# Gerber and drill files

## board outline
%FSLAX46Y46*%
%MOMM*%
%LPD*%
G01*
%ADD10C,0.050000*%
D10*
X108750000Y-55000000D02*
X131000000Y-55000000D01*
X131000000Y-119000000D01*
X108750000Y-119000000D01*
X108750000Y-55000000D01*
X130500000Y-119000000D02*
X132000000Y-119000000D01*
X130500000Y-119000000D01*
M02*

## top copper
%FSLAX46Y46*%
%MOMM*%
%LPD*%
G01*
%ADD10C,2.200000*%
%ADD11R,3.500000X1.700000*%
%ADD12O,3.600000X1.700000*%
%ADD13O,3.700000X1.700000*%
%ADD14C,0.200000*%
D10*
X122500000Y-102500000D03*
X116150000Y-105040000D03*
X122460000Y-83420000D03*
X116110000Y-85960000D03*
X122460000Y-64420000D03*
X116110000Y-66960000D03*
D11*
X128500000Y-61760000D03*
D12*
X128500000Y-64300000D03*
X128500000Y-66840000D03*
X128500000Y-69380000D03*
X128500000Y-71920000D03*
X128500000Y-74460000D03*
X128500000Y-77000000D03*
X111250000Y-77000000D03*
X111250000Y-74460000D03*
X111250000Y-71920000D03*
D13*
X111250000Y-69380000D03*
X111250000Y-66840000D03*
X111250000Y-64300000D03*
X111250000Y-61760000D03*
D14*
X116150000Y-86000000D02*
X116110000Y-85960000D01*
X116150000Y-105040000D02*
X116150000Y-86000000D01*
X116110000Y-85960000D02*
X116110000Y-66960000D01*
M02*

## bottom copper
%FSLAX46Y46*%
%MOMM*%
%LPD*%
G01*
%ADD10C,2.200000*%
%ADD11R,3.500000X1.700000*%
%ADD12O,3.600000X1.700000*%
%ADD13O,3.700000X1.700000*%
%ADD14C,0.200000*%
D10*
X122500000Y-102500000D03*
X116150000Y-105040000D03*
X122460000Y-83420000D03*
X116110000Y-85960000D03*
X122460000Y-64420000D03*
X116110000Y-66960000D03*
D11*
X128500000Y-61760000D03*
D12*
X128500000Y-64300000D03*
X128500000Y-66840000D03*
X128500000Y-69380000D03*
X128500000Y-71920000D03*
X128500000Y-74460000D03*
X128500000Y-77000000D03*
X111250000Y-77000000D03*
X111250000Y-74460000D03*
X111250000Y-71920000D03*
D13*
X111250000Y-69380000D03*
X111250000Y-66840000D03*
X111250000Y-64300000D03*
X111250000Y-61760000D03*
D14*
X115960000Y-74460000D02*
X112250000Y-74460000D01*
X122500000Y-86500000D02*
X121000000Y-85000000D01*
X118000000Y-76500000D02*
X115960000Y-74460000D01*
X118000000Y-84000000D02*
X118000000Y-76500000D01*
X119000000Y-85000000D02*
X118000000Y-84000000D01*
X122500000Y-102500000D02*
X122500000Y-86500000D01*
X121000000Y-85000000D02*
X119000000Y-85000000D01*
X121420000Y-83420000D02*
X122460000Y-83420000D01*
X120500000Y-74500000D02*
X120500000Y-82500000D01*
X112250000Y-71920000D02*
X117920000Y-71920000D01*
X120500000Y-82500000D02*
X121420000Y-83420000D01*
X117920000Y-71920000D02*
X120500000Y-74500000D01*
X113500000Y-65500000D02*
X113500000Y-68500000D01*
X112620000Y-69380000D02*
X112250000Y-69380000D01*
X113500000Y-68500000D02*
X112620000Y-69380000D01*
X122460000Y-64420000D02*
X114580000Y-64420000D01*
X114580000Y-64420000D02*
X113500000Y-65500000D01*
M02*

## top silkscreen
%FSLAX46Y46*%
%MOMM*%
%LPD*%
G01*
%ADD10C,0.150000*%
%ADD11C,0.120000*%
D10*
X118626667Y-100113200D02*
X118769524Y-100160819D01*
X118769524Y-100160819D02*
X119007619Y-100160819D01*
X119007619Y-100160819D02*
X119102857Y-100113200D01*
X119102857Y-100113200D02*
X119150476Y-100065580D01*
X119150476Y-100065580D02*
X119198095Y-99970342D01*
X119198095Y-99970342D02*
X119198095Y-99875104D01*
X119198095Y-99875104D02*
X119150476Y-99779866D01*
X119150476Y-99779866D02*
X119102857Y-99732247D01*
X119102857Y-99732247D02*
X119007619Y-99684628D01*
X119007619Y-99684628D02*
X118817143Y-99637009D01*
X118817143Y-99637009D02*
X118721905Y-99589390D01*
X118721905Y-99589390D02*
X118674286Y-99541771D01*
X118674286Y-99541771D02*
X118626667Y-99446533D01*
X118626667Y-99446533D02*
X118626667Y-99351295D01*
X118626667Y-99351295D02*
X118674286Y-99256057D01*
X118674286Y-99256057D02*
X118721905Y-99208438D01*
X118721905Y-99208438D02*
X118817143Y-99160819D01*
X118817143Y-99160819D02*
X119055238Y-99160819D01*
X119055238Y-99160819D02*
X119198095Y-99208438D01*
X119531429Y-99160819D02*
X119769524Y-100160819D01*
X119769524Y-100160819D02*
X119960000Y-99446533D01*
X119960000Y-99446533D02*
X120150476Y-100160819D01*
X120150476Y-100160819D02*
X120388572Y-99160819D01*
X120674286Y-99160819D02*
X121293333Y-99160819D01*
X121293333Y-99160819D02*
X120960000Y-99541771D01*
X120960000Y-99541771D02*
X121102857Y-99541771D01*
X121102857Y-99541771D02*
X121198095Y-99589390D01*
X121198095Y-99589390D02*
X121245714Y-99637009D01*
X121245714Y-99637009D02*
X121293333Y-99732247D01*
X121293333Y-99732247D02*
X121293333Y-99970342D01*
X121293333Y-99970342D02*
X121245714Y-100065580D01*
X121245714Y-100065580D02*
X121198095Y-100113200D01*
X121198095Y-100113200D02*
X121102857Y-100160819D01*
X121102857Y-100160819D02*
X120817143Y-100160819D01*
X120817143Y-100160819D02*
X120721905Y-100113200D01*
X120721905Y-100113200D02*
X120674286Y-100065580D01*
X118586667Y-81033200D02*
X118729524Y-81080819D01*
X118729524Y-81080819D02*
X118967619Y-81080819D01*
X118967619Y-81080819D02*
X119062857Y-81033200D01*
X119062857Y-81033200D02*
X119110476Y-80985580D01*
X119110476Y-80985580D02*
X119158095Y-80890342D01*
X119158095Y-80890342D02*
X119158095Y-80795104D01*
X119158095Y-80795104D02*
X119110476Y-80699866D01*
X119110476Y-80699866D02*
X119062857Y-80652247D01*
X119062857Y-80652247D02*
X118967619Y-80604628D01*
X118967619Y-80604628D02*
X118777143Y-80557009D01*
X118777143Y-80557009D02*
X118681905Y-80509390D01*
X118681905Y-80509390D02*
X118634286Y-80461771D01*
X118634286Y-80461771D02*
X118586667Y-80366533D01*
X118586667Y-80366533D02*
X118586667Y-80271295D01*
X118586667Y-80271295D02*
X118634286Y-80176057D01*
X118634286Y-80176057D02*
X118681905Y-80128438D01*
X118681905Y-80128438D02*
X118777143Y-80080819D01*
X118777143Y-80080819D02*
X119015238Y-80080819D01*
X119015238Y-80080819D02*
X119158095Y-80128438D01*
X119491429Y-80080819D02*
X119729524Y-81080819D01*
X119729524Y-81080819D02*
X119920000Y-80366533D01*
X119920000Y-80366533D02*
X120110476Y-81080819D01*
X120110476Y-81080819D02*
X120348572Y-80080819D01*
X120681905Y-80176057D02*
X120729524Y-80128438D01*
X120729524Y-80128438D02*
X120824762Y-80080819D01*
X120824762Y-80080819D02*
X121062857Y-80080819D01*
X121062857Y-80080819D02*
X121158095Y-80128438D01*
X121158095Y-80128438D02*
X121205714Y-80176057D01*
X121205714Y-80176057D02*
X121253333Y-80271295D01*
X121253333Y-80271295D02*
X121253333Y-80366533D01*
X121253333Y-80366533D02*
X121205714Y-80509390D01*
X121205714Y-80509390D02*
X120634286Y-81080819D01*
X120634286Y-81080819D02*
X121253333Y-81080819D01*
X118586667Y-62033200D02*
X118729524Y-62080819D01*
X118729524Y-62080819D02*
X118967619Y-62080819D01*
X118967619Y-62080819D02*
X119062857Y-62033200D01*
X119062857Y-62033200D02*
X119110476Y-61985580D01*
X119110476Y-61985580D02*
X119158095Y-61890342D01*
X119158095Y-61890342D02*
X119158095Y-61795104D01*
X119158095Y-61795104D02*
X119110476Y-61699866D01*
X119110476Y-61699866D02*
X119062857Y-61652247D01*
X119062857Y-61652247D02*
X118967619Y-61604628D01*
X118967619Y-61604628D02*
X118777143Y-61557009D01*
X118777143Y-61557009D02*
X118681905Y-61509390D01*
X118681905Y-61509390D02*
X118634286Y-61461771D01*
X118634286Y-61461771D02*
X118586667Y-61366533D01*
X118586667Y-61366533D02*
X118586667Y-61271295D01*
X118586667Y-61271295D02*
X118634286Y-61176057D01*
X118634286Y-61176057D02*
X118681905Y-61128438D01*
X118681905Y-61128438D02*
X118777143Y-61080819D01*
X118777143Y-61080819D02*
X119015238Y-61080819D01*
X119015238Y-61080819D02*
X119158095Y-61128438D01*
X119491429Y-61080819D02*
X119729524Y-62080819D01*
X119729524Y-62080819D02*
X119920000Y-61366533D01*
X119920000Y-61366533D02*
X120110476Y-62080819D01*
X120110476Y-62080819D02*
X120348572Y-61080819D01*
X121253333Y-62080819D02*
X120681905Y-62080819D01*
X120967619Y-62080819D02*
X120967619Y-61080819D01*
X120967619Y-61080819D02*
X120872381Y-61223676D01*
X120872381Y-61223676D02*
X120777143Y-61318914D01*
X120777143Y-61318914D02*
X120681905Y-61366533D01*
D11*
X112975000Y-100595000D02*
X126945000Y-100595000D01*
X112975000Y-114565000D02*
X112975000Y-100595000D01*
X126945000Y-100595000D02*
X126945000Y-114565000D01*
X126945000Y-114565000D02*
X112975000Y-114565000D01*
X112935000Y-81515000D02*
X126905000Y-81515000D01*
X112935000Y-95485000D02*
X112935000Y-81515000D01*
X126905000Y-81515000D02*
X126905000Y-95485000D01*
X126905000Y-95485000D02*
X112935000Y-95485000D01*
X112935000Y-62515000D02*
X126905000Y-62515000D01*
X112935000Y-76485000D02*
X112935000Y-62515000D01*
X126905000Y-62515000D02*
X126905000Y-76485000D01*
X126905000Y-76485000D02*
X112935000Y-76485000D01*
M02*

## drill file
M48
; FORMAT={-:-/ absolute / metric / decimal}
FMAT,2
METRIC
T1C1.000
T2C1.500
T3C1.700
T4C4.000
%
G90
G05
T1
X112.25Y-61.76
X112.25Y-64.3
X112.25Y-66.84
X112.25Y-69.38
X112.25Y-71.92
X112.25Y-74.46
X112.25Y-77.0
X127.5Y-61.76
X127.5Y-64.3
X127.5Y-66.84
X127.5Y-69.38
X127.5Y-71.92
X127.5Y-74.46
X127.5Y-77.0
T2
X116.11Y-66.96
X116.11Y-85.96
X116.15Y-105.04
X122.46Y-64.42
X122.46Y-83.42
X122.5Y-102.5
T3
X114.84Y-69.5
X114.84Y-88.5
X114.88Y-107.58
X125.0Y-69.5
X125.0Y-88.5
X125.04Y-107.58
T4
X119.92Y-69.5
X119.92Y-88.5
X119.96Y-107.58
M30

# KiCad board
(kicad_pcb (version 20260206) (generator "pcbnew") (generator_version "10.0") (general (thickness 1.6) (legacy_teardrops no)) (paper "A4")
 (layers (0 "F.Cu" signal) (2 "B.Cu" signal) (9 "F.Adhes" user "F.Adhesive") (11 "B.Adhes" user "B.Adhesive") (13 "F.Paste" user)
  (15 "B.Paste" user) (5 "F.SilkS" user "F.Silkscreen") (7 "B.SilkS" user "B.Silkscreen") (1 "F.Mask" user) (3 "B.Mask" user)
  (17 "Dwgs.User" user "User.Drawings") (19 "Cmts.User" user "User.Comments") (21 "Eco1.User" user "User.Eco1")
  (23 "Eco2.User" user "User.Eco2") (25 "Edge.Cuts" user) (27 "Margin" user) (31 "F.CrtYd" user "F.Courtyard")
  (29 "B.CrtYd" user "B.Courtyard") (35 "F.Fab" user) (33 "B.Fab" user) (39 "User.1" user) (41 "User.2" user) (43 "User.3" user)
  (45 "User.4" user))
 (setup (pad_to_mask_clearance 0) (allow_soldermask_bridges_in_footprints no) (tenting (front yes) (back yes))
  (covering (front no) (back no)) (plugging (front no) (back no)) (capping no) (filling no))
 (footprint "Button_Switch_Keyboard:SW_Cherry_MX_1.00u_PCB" (layer "F.Cu") (at 122.5 102.5)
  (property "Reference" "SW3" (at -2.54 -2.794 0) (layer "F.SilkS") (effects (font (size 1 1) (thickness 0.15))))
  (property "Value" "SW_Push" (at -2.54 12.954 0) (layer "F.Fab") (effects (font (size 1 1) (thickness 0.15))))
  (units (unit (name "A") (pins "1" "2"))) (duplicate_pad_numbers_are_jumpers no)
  (fp_line (start -9.525 -1.905) (end 4.445 -1.905) (stroke (width 0.12) (type solid)) (layer "F.SilkS"))
  (fp_line (start -9.525 12.065) (end -9.525 -1.905) (stroke (width 0.12) (type solid)) (layer "F.SilkS"))
  (fp_line (start 4.445 -1.905) (end 4.445 12.065) (stroke (width 0.12) (type solid)) (layer "F.SilkS"))
  (fp_line (start 4.445 12.065) (end -9.525 12.065) (stroke (width 0.12) (type solid)) (layer "F.SilkS"))
  (pad "" np_thru_hole circle (at -7.62 5.08) (size 1.7 1.7) (drill 1.7) (layers "*.Cu" "*.Mask"))
  (pad "" np_thru_hole circle (at -2.54 5.08) (size 4 4) (drill 4) (layers "*.Cu" "*.Mask"))
  (pad "" np_thru_hole circle (at 2.54 5.08) (size 1.7 1.7) (drill 1.7) (layers "*.Cu" "*.Mask"))
  (pad "1" thru_hole circle (at 0 0) (size 2.2 2.2) (drill 1.5) (layers "*.Cu" "*.Mask") (remove_unused_layers no)
   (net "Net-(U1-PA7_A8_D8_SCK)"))
  (pad "2" thru_hole circle (at -6.35 2.54) (size 2.2 2.2) (drill 1.5) (layers "*.Cu" "*.Mask") (remove_unused_layers no) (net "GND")))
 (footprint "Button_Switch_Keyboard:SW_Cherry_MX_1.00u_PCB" (layer "F.Cu") (at 122.46 83.42)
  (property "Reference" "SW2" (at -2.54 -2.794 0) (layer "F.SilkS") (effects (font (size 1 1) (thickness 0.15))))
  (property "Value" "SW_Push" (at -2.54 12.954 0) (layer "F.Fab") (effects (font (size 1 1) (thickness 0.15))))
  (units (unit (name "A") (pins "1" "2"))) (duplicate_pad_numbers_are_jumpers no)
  (fp_line (start -9.525 -1.905) (end 4.445 -1.905) (stroke (width 0.12) (type solid)) (layer "F.SilkS"))
  (fp_line (start -9.525 12.065) (end -9.525 -1.905) (stroke (width 0.12) (type solid)) (layer "F.SilkS"))
  (fp_line (start 4.445 -1.905) (end 4.445 12.065) (stroke (width 0.12) (type solid)) (layer "F.SilkS"))
  (fp_line (start 4.445 12.065) (end -9.525 12.065) (stroke (width 0.12) (type solid)) (layer "F.SilkS"))
  (pad "" np_thru_hole circle (at -7.62 5.08) (size 1.7 1.7) (drill 1.7) (layers "*.Cu" "*.Mask"))
  (pad "" np_thru_hole circle (at -2.54 5.08) (size 4 4) (drill 4) (layers "*.Cu" "*.Mask"))
  (pad "" np_thru_hole circle (at 2.54 5.08) (size 1.7 1.7) (drill 1.7) (layers "*.Cu" "*.Mask"))
  (pad "1" thru_hole circle (at 0 0) (size 2.2 2.2) (drill 1.5) (layers "*.Cu" "*.Mask") (remove_unused_layers no)
   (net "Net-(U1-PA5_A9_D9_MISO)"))
  (pad "2" thru_hole circle (at -6.35 2.54) (size 2.2 2.2) (drill 1.5) (layers "*.Cu" "*.Mask") (remove_unused_layers no) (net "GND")))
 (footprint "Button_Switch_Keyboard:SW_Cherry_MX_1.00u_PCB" (layer "F.Cu") (at 122.46 64.42)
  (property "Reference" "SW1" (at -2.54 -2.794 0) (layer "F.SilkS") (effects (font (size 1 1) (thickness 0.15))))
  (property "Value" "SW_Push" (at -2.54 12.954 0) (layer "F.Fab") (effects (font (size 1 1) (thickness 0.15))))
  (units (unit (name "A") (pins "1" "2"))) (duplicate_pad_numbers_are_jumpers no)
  (fp_line (start -9.525 -1.905) (end 4.445 -1.905) (stroke (width 0.12) (type solid)) (layer "F.SilkS"))
  (fp_line (start -9.525 12.065) (end -9.525 -1.905) (stroke (width 0.12) (type solid)) (layer "F.SilkS"))
  (fp_line (start 4.445 -1.905) (end 4.445 12.065) (stroke (width 0.12) (type solid)) (layer "F.SilkS"))
  (fp_line (start 4.445 12.065) (end -9.525 12.065) (stroke (width 0.12) (type solid)) (layer "F.SilkS"))
  (pad "" np_thru_hole circle (at -7.62 5.08) (size 1.7 1.7) (drill 1.7) (layers "*.Cu" "*.Mask"))
  (pad "" np_thru_hole circle (at -2.54 5.08) (size 4 4) (drill 4) (layers "*.Cu" "*.Mask"))
  (pad "" np_thru_hole circle (at 2.54 5.08) (size 1.7 1.7) (drill 1.7) (layers "*.Cu" "*.Mask"))
  (pad "1" thru_hole circle (at 0 0) (size 2.2 2.2) (drill 1.5) (layers "*.Cu" "*.Mask") (remove_unused_layers no)
   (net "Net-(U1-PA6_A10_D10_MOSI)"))
  (pad "2" thru_hole circle (at -6.35 2.54) (size 2.2 2.2) (drill 1.5) (layers "*.Cu" "*.Mask") (remove_unused_layers no) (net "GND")))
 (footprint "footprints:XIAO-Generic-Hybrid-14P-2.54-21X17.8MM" (layer "B.Cu") (at 119.875 69.38 180)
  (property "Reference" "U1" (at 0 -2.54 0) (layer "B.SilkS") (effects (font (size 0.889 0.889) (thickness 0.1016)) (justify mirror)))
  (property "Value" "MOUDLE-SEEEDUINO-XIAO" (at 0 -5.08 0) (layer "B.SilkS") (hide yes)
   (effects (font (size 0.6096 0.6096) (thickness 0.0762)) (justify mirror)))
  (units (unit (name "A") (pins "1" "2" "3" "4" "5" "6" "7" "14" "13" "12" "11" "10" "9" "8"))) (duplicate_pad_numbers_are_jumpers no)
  (pad "1" thru_hole rect (at -7.625 7.62 180) (size 3.5 1.7) (drill 1 (offset -1 0)) (layers "*.Cu" "*.Mask") (remove_unused_layers no)
   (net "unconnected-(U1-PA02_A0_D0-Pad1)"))
  (pad "2" thru_hole oval (at -7.625 5.08 180) (size 3.6 1.7) (drill 1 (offset -1 0)) (layers "*.Cu" "*.Mask") (remove_unused_layers no)
   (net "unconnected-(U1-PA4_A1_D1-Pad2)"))
  (pad "3" thru_hole oval (at -7.625 2.54 180) (size 3.6 1.7) (drill 1 (offset -1 0)) (layers "*.Cu" "*.Mask") (remove_unused_layers no)
   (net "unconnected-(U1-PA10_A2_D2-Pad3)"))
  (pad "4" thru_hole oval (at -7.625 0 180) (size 3.6 1.7) (drill 1 (offset -1 0)) (layers "*.Cu" "*.Mask") (remove_unused_layers no)
   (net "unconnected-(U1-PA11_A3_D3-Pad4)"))
  (pad "5" thru_hole oval (at -7.625 -2.54 180) (size 3.6 1.7) (drill 1 (offset -1 0)) (layers "*.Cu" "*.Mask") (remove_unused_layers no)
   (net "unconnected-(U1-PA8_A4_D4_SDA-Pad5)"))
  (pad "6" thru_hole oval (at -7.625 -5.08) (size 3.6 1.7) (drill 1 (offset 1 0)) (layers "*.Cu" "*.Mask") (remove_unused_layers no)
   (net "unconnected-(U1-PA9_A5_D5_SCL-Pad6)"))
  (pad "7" thru_hole oval (at -7.625 -7.62 180) (size 3.6 1.7) (drill 1 (offset -1 0)) (layers "*.Cu" "*.Mask") (remove_unused_layers no)
   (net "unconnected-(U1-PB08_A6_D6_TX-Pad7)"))
  (pad "8" thru_hole oval (at 7.625 -7.62 180) (size 3.6 1.7) (drill 1 (offset 1 0)) (layers "*.Cu" "*.Mask") (remove_unused_layers no)
   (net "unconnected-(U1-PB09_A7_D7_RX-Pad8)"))
  (pad "9" thru_hole oval (at 7.625 -5.08 180) (size 3.6 1.7) (drill 1 (offset 1 0)) (layers "*.Cu" "*.Mask") (remove_unused_layers no)
   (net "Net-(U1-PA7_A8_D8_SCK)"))
  (pad "10" thru_hole oval (at 7.625 -2.54 180) (size 3.6 1.7) (drill 1 (offset 1 0)) (layers "*.Cu" "*.Mask") (remove_unused_layers no)
   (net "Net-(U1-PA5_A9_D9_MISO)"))
  (pad "11" thru_hole oval (at 7.625 0 180) (size 3.7 1.7) (drill 1 (offset 1 0)) (layers "*.Cu" "*.Mask") (remove_unused_layers no)
   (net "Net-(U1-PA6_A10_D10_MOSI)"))
  (pad "12" thru_hole oval (at 7.625 2.54 180) (size 3.7 1.7) (drill 1 (offset 1 0)) (layers "*.Cu" "*.Mask") (remove_unused_layers no)
   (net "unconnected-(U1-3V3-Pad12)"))
  (pad "13" thru_hole oval (at 7.625 5.08 180) (size 3.7 1.7) (drill 1 (offset 1 0)) (layers "*.Cu" "*.Mask") (remove_unused_layers no)
   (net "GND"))
  (pad "14" thru_hole oval (at 7.625 7.62 180) (size 3.7 1.7) (drill 1 (offset 1 0)) (layers "*.Cu" "*.Mask") (remove_unused_layers no)
   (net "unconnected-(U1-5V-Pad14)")))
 (gr_rect (start 108.75 55) (end 131 119) (stroke (width 0.05) (type default)) (fill no) (layer "Edge.Cuts"))
 (gr_rect (start 130.5 119) (end 132 119) (stroke (width 0.05) (type default)) (fill no) (layer "Edge.Cuts"))
 (segment (start 115.96 74.46) (end 112.25 74.46) (width 0.2) (layer "B.Cu") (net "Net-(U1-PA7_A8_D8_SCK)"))
 (segment (start 122.5 86.5) (end 121 85) (width 0.2) (layer "B.Cu") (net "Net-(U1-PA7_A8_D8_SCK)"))
 (segment (start 118 76.5) (end 115.96 74.46) (width 0.2) (layer "B.Cu") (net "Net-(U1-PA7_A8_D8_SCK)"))
 (segment (start 118 84) (end 118 76.5) (width 0.2) (layer "B.Cu") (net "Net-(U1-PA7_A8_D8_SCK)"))
 (segment (start 119 85) (end 118 84) (width 0.2) (layer "B.Cu") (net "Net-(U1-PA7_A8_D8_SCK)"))
 (segment (start 122.5 102.5) (end 122.5 86.5) (width 0.2) (layer "B.Cu") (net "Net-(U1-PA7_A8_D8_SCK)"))
 (segment (start 121 85) (end 119 85) (width 0.2) (layer "B.Cu") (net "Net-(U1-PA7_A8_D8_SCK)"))
 (segment (start 116.15 86) (end 116.11 85.96) (width 0.2) (layer "F.Cu") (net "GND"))
 (segment (start 116.15 105.04) (end 116.15 86) (width 0.2) (layer "F.Cu") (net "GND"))
 (segment (start 116.11 85.96) (end 116.11 66.96) (width 0.2) (layer "F.Cu") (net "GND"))
 (segment (start 121.42 83.42) (end 122.46 83.42) (width 0.2) (layer "B.Cu") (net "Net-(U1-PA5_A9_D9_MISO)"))
 (segment (start 120.5 74.5) (end 120.5 82.5) (width 0.2) (layer "B.Cu") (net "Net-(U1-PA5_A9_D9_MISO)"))
 (segment (start 112.25 71.92) (end 117.92 71.92) (width 0.2) (layer "B.Cu") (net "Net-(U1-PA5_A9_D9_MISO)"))
 (segment (start 120.5 82.5) (end 121.42 83.42) (width 0.2) (layer "B.Cu") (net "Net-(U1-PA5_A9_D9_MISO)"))
 (segment (start 117.92 71.92) (end 120.5 74.5) (width 0.2) (layer "B.Cu") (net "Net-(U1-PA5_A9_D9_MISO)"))
 (segment (start 113.5 65.5) (end 113.5 68.5) (width 0.2) (layer "B.Cu") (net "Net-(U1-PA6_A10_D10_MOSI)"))
 (segment (start 112.62 69.38) (end 112.25 69.38) (width 0.2) (layer "B.Cu") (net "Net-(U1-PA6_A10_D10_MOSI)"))
 (segment (start 113.5 68.5) (end 112.62 69.38) (width 0.2) (layer "B.Cu") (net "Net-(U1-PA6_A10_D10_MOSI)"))
 (segment (start 122.46 64.42) (end 114.58 64.42) (width 0.2) (layer "B.Cu") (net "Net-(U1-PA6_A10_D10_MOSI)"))
 (segment (start 114.58 64.42) (end 113.5 65.5) (width 0.2) (layer "B.Cu") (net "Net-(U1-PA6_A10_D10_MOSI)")))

